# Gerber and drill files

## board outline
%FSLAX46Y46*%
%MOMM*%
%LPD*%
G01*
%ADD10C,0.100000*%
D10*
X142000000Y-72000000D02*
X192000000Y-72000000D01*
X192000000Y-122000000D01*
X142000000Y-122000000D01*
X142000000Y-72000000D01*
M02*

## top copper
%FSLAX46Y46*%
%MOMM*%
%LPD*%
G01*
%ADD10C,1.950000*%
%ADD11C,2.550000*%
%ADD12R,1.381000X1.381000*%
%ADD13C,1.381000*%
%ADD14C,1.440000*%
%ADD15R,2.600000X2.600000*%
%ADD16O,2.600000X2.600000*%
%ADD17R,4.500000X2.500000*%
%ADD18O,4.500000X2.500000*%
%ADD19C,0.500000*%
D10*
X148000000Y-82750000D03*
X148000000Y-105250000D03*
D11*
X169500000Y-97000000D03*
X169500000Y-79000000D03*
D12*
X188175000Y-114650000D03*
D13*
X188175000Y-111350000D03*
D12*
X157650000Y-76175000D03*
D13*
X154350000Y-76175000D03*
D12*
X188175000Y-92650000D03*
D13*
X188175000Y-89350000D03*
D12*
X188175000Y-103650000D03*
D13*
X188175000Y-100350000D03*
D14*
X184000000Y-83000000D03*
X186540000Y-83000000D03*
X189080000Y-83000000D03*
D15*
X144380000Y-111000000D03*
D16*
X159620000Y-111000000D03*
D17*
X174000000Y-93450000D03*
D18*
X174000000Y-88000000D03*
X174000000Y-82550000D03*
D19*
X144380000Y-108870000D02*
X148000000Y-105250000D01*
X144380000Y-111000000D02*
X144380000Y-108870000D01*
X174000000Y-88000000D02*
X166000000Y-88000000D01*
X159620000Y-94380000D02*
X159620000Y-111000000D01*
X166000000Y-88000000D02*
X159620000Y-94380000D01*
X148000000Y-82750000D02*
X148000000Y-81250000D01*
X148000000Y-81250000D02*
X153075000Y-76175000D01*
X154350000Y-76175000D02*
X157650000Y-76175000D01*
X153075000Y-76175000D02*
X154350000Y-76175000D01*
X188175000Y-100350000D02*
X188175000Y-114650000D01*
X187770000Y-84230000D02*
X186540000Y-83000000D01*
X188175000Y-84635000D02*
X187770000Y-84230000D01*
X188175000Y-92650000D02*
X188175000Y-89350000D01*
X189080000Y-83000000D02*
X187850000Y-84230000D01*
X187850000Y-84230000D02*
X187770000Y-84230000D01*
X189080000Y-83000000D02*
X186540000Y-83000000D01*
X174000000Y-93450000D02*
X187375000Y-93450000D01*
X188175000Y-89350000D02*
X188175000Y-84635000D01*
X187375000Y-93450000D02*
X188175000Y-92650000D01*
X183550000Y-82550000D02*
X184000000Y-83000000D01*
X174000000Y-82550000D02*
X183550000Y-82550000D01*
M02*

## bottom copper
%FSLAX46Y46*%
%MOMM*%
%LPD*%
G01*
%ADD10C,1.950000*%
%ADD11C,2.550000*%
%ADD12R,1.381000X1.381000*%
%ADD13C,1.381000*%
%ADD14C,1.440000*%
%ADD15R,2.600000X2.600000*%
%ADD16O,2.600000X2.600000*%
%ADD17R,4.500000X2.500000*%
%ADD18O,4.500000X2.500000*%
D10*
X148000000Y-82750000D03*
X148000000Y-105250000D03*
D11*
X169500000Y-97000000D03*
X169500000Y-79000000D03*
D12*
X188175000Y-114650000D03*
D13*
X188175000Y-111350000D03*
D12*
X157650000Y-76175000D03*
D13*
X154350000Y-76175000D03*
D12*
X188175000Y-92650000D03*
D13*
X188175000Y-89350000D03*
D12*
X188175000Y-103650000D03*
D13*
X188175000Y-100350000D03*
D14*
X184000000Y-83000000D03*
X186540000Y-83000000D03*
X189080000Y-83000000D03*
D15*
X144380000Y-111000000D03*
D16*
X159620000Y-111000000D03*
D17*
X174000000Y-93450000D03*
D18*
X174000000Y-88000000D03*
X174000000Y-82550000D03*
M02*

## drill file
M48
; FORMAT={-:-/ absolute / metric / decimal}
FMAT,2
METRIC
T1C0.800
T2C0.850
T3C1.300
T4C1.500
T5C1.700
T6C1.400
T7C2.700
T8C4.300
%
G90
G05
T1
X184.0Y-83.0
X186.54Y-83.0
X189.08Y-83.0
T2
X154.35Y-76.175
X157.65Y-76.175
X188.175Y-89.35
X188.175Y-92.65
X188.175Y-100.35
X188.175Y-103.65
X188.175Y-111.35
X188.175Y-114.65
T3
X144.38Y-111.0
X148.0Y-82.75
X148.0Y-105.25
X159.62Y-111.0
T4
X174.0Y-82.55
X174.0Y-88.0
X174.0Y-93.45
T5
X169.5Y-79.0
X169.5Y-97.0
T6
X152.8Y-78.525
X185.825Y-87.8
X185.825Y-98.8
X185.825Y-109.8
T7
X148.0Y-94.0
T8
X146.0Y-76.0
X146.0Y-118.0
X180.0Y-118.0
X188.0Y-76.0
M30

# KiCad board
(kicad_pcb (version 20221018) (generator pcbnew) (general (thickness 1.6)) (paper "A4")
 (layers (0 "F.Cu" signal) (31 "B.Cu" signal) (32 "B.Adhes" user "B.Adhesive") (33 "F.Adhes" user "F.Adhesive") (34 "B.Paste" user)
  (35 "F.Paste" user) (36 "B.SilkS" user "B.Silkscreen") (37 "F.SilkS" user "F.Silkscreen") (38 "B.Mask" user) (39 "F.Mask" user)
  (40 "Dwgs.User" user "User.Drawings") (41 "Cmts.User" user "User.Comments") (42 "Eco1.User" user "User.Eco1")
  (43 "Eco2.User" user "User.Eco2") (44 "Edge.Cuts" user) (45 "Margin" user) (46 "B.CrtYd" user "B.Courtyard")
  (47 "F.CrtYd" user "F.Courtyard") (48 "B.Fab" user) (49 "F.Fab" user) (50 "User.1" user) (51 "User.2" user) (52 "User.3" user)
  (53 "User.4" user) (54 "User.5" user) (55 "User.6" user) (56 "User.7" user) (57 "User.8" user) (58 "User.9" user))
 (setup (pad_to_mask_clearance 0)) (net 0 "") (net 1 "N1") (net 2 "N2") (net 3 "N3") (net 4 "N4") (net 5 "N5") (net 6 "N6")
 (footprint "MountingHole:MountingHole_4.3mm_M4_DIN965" (layer "F.Cu") (at 146 118)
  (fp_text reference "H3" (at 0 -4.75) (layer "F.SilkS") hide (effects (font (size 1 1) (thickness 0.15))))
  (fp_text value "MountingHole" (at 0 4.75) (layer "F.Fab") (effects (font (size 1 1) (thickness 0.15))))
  (pad "" np_thru_hole circle (at 0 0) (size 4.3 4.3) (drill 4.3) (layers "*.Cu" "*.Mask")))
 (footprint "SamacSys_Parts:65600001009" (layer "F.Cu") (at 148 94 -90)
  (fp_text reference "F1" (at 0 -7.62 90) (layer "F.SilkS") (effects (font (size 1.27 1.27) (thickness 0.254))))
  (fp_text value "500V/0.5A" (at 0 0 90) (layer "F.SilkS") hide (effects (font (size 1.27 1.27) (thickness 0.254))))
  (pad "" np_thru_hole circle (at 0 0 270) (size 2.7 2.7) (drill 2.7) (layers "F&B.Cu" "*.Mask"))
  (pad "1" thru_hole circle (at -11.25 0 270) (size 1.95 1.95) (drill 1.3) (layers "*.Cu" "*.Mask") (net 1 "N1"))
  (pad "2" thru_hole circle (at 11.25 0 270) (size 1.95 1.95) (drill 1.3) (layers "*.Cu" "*.Mask") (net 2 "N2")))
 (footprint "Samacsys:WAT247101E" (layer "F.Cu") (at 169.5 97 90)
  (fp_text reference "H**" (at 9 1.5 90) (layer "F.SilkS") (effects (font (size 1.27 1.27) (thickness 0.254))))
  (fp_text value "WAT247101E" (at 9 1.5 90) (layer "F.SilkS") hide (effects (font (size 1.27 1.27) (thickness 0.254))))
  (pad "1" thru_hole circle (at 0 0 90) (size 2.55 2.55) (drill 1.7) (layers "*.Cu" "*.Mask"))
  (pad "2" thru_hole circle (at 18 0 90) (size 2.55 2.55) (drill 1.7) (layers "*.Cu" "*.Mask")))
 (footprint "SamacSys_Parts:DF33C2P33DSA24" (layer "F.Cu") (at 188.175 114.65 90)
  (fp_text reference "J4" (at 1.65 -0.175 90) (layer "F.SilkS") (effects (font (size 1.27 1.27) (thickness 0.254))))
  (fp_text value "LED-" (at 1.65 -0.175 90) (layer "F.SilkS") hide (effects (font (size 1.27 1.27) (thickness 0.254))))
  (pad "" np_thru_hole circle (at 4.85 -2.35 90) (size 1.4 1.4) (drill 1.4) (layers "*.Cu" "*.Mask"))
  (pad "1" thru_hole rect (at 0 0 90) (size 1.381 1.381) (drill 0.85) (layers "*.Cu" "*.Mask") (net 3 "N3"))
  (pad "2" thru_hole circle (at 3.3 0 90) (size 1.381 1.381) (drill 0.85) (layers "*.Cu" "*.Mask") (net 3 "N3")))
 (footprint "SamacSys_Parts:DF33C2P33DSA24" (layer "F.Cu") (at 157.65 76.175 180)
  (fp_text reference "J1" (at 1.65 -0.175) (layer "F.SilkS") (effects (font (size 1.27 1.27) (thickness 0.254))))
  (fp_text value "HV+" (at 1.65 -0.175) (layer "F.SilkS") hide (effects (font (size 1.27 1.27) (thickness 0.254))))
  (pad "" np_thru_hole circle (at 4.85 -2.35 180) (size 1.4 1.4) (drill 1.4) (layers "*.Cu" "*.Mask"))
  (pad "1" thru_hole rect (at 0 0 180) (size 1.381 1.381) (drill 0.85) (layers "*.Cu" "*.Mask") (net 1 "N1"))
  (pad "2" thru_hole circle (at 3.3 0 180) (size 1.381 1.381) (drill 0.85) (layers "*.Cu" "*.Mask") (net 1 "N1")))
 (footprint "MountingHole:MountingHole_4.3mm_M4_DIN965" (layer "F.Cu") (at 180 118)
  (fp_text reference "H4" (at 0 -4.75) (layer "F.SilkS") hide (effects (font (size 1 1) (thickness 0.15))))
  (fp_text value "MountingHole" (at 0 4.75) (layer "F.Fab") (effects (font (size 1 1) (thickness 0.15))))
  (pad "" np_thru_hole circle (at 0 0) (size 4.3 4.3) (drill 4.3) (layers "*.Cu" "*.Mask")))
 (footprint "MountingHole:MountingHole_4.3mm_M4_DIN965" (layer "F.Cu") (at 188 76)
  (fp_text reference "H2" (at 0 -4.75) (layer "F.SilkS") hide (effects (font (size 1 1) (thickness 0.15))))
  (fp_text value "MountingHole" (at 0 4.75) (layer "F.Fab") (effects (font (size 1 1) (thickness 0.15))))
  (pad "" np_thru_hole circle (at 0 0) (size 4.3 4.3) (drill 4.3) (layers "*.Cu" "*.Mask")))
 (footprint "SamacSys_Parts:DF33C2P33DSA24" (layer "F.Cu") (at 188.175 92.65 90)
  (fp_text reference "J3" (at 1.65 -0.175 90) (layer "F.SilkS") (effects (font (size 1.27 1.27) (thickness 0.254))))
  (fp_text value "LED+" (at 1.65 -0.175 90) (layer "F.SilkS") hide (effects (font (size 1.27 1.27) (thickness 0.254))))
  (pad "" np_thru_hole circle (at 4.85 -2.35 90) (size 1.4 1.4) (drill 1.4) (layers "*.Cu" "*.Mask"))
  (pad "1" thru_hole rect (at 0 0 90) (size 1.381 1.381) (drill 0.85) (layers "*.Cu" "*.Mask") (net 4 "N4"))
  (pad "2" thru_hole circle (at 3.3 0 90) (size 1.381 1.381) (drill 0.85) (layers "*.Cu" "*.Mask") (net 4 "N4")))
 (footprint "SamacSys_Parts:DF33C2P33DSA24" (layer "F.Cu") (at 188.175 103.65 90)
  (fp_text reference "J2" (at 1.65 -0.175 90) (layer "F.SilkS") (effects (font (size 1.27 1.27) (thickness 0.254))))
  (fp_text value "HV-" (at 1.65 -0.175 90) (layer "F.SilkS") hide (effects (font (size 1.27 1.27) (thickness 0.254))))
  (pad "" np_thru_hole circle (at 4.85 -2.35 90) (size 1.4 1.4) (drill 1.4) (layers "*.Cu" "*.Mask"))
  (pad "1" thru_hole rect (at 0 0 90) (size 1.381 1.381) (drill 0.85) (layers "*.Cu" "*.Mask") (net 3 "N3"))
  (pad "2" thru_hole circle (at 3.3 0 90) (size 1.381 1.381) (drill 0.85) (layers "*.Cu" "*.Mask") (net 3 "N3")))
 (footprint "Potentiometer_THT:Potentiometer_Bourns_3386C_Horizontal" (layer "F.Cu") (at 184 83 90)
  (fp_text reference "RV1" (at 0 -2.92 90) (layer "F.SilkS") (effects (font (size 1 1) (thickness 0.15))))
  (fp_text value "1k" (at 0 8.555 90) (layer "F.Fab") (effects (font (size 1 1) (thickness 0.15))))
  (pad "1" thru_hole circle (at 0 0 90) (size 1.44 1.44) (drill 0.8) (layers "*.Cu" "*.Mask") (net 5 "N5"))
  (pad "2" thru_hole circle (at 0 2.54 90) (size 1.44 1.44) (drill 0.8) (layers "*.Cu" "*.Mask") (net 4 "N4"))
  (pad "3" thru_hole circle (at 0 5.08 90) (size 1.44 1.44) (drill 0.8) (layers "*.Cu" "*.Mask") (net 4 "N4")))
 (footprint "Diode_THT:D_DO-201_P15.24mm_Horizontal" (layer "F.Cu") (at 144.38 111)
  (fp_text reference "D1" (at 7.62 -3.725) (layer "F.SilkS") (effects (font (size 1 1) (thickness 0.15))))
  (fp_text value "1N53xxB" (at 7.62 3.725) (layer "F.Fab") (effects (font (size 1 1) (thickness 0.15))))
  (pad "1" thru_hole rect (at 0 0) (size 2.6 2.6) (drill 1.3) (layers "*.Cu" "*.Mask") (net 2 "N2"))
  (pad "2" thru_hole oval (at 15.24 0) (size 2.6 2.6) (drill 1.3) (layers "*.Cu" "*.Mask") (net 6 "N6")))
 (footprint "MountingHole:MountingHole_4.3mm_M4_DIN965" (layer "F.Cu") (at 146 76)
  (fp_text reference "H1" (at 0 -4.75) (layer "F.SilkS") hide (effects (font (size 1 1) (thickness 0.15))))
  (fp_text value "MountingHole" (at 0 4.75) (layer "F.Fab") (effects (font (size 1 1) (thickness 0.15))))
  (pad "" np_thru_hole circle (at 0 0) (size 4.3 4.3) (drill 4.3) (layers "*.Cu" "*.Mask")))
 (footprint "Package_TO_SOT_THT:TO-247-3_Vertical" (layer "F.Cu") (at 174 93.45 90)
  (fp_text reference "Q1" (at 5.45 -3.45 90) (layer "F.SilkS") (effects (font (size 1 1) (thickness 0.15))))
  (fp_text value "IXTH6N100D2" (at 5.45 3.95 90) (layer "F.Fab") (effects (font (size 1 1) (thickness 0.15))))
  (pad "1" thru_hole rect (at 0 0 90) (size 2.5 4.5) (drill 1.5) (layers "*.Cu" "*.Mask") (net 4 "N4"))
  (pad "2" thru_hole oval (at 5.45 0 90) (size 2.5 4.5) (drill 1.5) (layers "*.Cu" "*.Mask") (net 6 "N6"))
  (pad "3" thru_hole oval (at 10.9 0 90) (size 2.5 4.5) (drill 1.5) (layers "*.Cu" "*.Mask") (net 5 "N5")))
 (gr_rect (start 142 72) (end 192 122) (stroke (width 0.1) (type default)) (fill none) (layer "Edge.Cuts"))
 (segment (start 144.38 108.87) (end 148 105.25) (width 0.5) (layer "F.Cu") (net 2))
 (segment (start 144.38 111) (end 144.38 108.87) (width 0.5) (layer "F.Cu") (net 2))
 (segment (start 174 88) (end 166 88) (width 0.5) (layer "F.Cu") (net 6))
 (segment (start 159.62 94.38) (end 159.62 111) (width 0.5) (layer "F.Cu") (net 6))
 (segment (start 166 88) (end 159.62 94.38) (width 0.5) (layer "F.Cu") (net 6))
 (segment (start 148 82.75) (end 148 81.25) (width 0.5) (layer "F.Cu") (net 1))
 (segment (start 148 81.25) (end 153.075 76.175) (width 0.5) (layer "F.Cu") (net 1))
 (segment (start 154.35 76.175) (end 157.65 76.175) (width 0.5) (layer "F.Cu") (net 1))
 (segment (start 153.075 76.175) (end 154.35 76.175) (width 0.5) (layer "F.Cu") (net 1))
 (segment (start 188.175 100.35) (end 188.175 114.65) (width 0.5) (layer "F.Cu") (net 3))
 (segment (start 187.77 84.23) (end 186.54 83) (width 0.5) (layer "F.Cu") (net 4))
 (segment (start 188.175 84.635) (end 187.77 84.23) (width 0.5) (layer "F.Cu") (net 4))
 (segment (start 188.175 92.65) (end 188.175 89.35) (width 0.5) (layer "F.Cu") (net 4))
 (segment (start 189.08 83) (end 187.85 84.23) (width 0.5) (layer "F.Cu") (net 4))
 (segment (start 187.85 84.23) (end 187.77 84.23) (width 0.5) (layer "F.Cu") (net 4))
 (segment (start 189.08 83) (end 186.54 83) (width 0.5) (layer "F.Cu") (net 4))
 (segment (start 174 93.45) (end 187.375 93.45) (width 0.5) (layer "F.Cu") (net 4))
 (segment (start 188.175 89.35) (end 188.175 84.635) (width 0.5) (layer "F.Cu") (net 4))
 (segment (start 187.375 93.45) (end 188.175 92.65) (width 0.5) (layer "F.Cu") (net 4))
 (segment (start 183.55 82.55) (end 184 83) (width 0.5) (layer "F.Cu") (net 5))
 (segment (start 174 82.55) (end 183.55 82.55) (width 0.5) (layer "F.Cu") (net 5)))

